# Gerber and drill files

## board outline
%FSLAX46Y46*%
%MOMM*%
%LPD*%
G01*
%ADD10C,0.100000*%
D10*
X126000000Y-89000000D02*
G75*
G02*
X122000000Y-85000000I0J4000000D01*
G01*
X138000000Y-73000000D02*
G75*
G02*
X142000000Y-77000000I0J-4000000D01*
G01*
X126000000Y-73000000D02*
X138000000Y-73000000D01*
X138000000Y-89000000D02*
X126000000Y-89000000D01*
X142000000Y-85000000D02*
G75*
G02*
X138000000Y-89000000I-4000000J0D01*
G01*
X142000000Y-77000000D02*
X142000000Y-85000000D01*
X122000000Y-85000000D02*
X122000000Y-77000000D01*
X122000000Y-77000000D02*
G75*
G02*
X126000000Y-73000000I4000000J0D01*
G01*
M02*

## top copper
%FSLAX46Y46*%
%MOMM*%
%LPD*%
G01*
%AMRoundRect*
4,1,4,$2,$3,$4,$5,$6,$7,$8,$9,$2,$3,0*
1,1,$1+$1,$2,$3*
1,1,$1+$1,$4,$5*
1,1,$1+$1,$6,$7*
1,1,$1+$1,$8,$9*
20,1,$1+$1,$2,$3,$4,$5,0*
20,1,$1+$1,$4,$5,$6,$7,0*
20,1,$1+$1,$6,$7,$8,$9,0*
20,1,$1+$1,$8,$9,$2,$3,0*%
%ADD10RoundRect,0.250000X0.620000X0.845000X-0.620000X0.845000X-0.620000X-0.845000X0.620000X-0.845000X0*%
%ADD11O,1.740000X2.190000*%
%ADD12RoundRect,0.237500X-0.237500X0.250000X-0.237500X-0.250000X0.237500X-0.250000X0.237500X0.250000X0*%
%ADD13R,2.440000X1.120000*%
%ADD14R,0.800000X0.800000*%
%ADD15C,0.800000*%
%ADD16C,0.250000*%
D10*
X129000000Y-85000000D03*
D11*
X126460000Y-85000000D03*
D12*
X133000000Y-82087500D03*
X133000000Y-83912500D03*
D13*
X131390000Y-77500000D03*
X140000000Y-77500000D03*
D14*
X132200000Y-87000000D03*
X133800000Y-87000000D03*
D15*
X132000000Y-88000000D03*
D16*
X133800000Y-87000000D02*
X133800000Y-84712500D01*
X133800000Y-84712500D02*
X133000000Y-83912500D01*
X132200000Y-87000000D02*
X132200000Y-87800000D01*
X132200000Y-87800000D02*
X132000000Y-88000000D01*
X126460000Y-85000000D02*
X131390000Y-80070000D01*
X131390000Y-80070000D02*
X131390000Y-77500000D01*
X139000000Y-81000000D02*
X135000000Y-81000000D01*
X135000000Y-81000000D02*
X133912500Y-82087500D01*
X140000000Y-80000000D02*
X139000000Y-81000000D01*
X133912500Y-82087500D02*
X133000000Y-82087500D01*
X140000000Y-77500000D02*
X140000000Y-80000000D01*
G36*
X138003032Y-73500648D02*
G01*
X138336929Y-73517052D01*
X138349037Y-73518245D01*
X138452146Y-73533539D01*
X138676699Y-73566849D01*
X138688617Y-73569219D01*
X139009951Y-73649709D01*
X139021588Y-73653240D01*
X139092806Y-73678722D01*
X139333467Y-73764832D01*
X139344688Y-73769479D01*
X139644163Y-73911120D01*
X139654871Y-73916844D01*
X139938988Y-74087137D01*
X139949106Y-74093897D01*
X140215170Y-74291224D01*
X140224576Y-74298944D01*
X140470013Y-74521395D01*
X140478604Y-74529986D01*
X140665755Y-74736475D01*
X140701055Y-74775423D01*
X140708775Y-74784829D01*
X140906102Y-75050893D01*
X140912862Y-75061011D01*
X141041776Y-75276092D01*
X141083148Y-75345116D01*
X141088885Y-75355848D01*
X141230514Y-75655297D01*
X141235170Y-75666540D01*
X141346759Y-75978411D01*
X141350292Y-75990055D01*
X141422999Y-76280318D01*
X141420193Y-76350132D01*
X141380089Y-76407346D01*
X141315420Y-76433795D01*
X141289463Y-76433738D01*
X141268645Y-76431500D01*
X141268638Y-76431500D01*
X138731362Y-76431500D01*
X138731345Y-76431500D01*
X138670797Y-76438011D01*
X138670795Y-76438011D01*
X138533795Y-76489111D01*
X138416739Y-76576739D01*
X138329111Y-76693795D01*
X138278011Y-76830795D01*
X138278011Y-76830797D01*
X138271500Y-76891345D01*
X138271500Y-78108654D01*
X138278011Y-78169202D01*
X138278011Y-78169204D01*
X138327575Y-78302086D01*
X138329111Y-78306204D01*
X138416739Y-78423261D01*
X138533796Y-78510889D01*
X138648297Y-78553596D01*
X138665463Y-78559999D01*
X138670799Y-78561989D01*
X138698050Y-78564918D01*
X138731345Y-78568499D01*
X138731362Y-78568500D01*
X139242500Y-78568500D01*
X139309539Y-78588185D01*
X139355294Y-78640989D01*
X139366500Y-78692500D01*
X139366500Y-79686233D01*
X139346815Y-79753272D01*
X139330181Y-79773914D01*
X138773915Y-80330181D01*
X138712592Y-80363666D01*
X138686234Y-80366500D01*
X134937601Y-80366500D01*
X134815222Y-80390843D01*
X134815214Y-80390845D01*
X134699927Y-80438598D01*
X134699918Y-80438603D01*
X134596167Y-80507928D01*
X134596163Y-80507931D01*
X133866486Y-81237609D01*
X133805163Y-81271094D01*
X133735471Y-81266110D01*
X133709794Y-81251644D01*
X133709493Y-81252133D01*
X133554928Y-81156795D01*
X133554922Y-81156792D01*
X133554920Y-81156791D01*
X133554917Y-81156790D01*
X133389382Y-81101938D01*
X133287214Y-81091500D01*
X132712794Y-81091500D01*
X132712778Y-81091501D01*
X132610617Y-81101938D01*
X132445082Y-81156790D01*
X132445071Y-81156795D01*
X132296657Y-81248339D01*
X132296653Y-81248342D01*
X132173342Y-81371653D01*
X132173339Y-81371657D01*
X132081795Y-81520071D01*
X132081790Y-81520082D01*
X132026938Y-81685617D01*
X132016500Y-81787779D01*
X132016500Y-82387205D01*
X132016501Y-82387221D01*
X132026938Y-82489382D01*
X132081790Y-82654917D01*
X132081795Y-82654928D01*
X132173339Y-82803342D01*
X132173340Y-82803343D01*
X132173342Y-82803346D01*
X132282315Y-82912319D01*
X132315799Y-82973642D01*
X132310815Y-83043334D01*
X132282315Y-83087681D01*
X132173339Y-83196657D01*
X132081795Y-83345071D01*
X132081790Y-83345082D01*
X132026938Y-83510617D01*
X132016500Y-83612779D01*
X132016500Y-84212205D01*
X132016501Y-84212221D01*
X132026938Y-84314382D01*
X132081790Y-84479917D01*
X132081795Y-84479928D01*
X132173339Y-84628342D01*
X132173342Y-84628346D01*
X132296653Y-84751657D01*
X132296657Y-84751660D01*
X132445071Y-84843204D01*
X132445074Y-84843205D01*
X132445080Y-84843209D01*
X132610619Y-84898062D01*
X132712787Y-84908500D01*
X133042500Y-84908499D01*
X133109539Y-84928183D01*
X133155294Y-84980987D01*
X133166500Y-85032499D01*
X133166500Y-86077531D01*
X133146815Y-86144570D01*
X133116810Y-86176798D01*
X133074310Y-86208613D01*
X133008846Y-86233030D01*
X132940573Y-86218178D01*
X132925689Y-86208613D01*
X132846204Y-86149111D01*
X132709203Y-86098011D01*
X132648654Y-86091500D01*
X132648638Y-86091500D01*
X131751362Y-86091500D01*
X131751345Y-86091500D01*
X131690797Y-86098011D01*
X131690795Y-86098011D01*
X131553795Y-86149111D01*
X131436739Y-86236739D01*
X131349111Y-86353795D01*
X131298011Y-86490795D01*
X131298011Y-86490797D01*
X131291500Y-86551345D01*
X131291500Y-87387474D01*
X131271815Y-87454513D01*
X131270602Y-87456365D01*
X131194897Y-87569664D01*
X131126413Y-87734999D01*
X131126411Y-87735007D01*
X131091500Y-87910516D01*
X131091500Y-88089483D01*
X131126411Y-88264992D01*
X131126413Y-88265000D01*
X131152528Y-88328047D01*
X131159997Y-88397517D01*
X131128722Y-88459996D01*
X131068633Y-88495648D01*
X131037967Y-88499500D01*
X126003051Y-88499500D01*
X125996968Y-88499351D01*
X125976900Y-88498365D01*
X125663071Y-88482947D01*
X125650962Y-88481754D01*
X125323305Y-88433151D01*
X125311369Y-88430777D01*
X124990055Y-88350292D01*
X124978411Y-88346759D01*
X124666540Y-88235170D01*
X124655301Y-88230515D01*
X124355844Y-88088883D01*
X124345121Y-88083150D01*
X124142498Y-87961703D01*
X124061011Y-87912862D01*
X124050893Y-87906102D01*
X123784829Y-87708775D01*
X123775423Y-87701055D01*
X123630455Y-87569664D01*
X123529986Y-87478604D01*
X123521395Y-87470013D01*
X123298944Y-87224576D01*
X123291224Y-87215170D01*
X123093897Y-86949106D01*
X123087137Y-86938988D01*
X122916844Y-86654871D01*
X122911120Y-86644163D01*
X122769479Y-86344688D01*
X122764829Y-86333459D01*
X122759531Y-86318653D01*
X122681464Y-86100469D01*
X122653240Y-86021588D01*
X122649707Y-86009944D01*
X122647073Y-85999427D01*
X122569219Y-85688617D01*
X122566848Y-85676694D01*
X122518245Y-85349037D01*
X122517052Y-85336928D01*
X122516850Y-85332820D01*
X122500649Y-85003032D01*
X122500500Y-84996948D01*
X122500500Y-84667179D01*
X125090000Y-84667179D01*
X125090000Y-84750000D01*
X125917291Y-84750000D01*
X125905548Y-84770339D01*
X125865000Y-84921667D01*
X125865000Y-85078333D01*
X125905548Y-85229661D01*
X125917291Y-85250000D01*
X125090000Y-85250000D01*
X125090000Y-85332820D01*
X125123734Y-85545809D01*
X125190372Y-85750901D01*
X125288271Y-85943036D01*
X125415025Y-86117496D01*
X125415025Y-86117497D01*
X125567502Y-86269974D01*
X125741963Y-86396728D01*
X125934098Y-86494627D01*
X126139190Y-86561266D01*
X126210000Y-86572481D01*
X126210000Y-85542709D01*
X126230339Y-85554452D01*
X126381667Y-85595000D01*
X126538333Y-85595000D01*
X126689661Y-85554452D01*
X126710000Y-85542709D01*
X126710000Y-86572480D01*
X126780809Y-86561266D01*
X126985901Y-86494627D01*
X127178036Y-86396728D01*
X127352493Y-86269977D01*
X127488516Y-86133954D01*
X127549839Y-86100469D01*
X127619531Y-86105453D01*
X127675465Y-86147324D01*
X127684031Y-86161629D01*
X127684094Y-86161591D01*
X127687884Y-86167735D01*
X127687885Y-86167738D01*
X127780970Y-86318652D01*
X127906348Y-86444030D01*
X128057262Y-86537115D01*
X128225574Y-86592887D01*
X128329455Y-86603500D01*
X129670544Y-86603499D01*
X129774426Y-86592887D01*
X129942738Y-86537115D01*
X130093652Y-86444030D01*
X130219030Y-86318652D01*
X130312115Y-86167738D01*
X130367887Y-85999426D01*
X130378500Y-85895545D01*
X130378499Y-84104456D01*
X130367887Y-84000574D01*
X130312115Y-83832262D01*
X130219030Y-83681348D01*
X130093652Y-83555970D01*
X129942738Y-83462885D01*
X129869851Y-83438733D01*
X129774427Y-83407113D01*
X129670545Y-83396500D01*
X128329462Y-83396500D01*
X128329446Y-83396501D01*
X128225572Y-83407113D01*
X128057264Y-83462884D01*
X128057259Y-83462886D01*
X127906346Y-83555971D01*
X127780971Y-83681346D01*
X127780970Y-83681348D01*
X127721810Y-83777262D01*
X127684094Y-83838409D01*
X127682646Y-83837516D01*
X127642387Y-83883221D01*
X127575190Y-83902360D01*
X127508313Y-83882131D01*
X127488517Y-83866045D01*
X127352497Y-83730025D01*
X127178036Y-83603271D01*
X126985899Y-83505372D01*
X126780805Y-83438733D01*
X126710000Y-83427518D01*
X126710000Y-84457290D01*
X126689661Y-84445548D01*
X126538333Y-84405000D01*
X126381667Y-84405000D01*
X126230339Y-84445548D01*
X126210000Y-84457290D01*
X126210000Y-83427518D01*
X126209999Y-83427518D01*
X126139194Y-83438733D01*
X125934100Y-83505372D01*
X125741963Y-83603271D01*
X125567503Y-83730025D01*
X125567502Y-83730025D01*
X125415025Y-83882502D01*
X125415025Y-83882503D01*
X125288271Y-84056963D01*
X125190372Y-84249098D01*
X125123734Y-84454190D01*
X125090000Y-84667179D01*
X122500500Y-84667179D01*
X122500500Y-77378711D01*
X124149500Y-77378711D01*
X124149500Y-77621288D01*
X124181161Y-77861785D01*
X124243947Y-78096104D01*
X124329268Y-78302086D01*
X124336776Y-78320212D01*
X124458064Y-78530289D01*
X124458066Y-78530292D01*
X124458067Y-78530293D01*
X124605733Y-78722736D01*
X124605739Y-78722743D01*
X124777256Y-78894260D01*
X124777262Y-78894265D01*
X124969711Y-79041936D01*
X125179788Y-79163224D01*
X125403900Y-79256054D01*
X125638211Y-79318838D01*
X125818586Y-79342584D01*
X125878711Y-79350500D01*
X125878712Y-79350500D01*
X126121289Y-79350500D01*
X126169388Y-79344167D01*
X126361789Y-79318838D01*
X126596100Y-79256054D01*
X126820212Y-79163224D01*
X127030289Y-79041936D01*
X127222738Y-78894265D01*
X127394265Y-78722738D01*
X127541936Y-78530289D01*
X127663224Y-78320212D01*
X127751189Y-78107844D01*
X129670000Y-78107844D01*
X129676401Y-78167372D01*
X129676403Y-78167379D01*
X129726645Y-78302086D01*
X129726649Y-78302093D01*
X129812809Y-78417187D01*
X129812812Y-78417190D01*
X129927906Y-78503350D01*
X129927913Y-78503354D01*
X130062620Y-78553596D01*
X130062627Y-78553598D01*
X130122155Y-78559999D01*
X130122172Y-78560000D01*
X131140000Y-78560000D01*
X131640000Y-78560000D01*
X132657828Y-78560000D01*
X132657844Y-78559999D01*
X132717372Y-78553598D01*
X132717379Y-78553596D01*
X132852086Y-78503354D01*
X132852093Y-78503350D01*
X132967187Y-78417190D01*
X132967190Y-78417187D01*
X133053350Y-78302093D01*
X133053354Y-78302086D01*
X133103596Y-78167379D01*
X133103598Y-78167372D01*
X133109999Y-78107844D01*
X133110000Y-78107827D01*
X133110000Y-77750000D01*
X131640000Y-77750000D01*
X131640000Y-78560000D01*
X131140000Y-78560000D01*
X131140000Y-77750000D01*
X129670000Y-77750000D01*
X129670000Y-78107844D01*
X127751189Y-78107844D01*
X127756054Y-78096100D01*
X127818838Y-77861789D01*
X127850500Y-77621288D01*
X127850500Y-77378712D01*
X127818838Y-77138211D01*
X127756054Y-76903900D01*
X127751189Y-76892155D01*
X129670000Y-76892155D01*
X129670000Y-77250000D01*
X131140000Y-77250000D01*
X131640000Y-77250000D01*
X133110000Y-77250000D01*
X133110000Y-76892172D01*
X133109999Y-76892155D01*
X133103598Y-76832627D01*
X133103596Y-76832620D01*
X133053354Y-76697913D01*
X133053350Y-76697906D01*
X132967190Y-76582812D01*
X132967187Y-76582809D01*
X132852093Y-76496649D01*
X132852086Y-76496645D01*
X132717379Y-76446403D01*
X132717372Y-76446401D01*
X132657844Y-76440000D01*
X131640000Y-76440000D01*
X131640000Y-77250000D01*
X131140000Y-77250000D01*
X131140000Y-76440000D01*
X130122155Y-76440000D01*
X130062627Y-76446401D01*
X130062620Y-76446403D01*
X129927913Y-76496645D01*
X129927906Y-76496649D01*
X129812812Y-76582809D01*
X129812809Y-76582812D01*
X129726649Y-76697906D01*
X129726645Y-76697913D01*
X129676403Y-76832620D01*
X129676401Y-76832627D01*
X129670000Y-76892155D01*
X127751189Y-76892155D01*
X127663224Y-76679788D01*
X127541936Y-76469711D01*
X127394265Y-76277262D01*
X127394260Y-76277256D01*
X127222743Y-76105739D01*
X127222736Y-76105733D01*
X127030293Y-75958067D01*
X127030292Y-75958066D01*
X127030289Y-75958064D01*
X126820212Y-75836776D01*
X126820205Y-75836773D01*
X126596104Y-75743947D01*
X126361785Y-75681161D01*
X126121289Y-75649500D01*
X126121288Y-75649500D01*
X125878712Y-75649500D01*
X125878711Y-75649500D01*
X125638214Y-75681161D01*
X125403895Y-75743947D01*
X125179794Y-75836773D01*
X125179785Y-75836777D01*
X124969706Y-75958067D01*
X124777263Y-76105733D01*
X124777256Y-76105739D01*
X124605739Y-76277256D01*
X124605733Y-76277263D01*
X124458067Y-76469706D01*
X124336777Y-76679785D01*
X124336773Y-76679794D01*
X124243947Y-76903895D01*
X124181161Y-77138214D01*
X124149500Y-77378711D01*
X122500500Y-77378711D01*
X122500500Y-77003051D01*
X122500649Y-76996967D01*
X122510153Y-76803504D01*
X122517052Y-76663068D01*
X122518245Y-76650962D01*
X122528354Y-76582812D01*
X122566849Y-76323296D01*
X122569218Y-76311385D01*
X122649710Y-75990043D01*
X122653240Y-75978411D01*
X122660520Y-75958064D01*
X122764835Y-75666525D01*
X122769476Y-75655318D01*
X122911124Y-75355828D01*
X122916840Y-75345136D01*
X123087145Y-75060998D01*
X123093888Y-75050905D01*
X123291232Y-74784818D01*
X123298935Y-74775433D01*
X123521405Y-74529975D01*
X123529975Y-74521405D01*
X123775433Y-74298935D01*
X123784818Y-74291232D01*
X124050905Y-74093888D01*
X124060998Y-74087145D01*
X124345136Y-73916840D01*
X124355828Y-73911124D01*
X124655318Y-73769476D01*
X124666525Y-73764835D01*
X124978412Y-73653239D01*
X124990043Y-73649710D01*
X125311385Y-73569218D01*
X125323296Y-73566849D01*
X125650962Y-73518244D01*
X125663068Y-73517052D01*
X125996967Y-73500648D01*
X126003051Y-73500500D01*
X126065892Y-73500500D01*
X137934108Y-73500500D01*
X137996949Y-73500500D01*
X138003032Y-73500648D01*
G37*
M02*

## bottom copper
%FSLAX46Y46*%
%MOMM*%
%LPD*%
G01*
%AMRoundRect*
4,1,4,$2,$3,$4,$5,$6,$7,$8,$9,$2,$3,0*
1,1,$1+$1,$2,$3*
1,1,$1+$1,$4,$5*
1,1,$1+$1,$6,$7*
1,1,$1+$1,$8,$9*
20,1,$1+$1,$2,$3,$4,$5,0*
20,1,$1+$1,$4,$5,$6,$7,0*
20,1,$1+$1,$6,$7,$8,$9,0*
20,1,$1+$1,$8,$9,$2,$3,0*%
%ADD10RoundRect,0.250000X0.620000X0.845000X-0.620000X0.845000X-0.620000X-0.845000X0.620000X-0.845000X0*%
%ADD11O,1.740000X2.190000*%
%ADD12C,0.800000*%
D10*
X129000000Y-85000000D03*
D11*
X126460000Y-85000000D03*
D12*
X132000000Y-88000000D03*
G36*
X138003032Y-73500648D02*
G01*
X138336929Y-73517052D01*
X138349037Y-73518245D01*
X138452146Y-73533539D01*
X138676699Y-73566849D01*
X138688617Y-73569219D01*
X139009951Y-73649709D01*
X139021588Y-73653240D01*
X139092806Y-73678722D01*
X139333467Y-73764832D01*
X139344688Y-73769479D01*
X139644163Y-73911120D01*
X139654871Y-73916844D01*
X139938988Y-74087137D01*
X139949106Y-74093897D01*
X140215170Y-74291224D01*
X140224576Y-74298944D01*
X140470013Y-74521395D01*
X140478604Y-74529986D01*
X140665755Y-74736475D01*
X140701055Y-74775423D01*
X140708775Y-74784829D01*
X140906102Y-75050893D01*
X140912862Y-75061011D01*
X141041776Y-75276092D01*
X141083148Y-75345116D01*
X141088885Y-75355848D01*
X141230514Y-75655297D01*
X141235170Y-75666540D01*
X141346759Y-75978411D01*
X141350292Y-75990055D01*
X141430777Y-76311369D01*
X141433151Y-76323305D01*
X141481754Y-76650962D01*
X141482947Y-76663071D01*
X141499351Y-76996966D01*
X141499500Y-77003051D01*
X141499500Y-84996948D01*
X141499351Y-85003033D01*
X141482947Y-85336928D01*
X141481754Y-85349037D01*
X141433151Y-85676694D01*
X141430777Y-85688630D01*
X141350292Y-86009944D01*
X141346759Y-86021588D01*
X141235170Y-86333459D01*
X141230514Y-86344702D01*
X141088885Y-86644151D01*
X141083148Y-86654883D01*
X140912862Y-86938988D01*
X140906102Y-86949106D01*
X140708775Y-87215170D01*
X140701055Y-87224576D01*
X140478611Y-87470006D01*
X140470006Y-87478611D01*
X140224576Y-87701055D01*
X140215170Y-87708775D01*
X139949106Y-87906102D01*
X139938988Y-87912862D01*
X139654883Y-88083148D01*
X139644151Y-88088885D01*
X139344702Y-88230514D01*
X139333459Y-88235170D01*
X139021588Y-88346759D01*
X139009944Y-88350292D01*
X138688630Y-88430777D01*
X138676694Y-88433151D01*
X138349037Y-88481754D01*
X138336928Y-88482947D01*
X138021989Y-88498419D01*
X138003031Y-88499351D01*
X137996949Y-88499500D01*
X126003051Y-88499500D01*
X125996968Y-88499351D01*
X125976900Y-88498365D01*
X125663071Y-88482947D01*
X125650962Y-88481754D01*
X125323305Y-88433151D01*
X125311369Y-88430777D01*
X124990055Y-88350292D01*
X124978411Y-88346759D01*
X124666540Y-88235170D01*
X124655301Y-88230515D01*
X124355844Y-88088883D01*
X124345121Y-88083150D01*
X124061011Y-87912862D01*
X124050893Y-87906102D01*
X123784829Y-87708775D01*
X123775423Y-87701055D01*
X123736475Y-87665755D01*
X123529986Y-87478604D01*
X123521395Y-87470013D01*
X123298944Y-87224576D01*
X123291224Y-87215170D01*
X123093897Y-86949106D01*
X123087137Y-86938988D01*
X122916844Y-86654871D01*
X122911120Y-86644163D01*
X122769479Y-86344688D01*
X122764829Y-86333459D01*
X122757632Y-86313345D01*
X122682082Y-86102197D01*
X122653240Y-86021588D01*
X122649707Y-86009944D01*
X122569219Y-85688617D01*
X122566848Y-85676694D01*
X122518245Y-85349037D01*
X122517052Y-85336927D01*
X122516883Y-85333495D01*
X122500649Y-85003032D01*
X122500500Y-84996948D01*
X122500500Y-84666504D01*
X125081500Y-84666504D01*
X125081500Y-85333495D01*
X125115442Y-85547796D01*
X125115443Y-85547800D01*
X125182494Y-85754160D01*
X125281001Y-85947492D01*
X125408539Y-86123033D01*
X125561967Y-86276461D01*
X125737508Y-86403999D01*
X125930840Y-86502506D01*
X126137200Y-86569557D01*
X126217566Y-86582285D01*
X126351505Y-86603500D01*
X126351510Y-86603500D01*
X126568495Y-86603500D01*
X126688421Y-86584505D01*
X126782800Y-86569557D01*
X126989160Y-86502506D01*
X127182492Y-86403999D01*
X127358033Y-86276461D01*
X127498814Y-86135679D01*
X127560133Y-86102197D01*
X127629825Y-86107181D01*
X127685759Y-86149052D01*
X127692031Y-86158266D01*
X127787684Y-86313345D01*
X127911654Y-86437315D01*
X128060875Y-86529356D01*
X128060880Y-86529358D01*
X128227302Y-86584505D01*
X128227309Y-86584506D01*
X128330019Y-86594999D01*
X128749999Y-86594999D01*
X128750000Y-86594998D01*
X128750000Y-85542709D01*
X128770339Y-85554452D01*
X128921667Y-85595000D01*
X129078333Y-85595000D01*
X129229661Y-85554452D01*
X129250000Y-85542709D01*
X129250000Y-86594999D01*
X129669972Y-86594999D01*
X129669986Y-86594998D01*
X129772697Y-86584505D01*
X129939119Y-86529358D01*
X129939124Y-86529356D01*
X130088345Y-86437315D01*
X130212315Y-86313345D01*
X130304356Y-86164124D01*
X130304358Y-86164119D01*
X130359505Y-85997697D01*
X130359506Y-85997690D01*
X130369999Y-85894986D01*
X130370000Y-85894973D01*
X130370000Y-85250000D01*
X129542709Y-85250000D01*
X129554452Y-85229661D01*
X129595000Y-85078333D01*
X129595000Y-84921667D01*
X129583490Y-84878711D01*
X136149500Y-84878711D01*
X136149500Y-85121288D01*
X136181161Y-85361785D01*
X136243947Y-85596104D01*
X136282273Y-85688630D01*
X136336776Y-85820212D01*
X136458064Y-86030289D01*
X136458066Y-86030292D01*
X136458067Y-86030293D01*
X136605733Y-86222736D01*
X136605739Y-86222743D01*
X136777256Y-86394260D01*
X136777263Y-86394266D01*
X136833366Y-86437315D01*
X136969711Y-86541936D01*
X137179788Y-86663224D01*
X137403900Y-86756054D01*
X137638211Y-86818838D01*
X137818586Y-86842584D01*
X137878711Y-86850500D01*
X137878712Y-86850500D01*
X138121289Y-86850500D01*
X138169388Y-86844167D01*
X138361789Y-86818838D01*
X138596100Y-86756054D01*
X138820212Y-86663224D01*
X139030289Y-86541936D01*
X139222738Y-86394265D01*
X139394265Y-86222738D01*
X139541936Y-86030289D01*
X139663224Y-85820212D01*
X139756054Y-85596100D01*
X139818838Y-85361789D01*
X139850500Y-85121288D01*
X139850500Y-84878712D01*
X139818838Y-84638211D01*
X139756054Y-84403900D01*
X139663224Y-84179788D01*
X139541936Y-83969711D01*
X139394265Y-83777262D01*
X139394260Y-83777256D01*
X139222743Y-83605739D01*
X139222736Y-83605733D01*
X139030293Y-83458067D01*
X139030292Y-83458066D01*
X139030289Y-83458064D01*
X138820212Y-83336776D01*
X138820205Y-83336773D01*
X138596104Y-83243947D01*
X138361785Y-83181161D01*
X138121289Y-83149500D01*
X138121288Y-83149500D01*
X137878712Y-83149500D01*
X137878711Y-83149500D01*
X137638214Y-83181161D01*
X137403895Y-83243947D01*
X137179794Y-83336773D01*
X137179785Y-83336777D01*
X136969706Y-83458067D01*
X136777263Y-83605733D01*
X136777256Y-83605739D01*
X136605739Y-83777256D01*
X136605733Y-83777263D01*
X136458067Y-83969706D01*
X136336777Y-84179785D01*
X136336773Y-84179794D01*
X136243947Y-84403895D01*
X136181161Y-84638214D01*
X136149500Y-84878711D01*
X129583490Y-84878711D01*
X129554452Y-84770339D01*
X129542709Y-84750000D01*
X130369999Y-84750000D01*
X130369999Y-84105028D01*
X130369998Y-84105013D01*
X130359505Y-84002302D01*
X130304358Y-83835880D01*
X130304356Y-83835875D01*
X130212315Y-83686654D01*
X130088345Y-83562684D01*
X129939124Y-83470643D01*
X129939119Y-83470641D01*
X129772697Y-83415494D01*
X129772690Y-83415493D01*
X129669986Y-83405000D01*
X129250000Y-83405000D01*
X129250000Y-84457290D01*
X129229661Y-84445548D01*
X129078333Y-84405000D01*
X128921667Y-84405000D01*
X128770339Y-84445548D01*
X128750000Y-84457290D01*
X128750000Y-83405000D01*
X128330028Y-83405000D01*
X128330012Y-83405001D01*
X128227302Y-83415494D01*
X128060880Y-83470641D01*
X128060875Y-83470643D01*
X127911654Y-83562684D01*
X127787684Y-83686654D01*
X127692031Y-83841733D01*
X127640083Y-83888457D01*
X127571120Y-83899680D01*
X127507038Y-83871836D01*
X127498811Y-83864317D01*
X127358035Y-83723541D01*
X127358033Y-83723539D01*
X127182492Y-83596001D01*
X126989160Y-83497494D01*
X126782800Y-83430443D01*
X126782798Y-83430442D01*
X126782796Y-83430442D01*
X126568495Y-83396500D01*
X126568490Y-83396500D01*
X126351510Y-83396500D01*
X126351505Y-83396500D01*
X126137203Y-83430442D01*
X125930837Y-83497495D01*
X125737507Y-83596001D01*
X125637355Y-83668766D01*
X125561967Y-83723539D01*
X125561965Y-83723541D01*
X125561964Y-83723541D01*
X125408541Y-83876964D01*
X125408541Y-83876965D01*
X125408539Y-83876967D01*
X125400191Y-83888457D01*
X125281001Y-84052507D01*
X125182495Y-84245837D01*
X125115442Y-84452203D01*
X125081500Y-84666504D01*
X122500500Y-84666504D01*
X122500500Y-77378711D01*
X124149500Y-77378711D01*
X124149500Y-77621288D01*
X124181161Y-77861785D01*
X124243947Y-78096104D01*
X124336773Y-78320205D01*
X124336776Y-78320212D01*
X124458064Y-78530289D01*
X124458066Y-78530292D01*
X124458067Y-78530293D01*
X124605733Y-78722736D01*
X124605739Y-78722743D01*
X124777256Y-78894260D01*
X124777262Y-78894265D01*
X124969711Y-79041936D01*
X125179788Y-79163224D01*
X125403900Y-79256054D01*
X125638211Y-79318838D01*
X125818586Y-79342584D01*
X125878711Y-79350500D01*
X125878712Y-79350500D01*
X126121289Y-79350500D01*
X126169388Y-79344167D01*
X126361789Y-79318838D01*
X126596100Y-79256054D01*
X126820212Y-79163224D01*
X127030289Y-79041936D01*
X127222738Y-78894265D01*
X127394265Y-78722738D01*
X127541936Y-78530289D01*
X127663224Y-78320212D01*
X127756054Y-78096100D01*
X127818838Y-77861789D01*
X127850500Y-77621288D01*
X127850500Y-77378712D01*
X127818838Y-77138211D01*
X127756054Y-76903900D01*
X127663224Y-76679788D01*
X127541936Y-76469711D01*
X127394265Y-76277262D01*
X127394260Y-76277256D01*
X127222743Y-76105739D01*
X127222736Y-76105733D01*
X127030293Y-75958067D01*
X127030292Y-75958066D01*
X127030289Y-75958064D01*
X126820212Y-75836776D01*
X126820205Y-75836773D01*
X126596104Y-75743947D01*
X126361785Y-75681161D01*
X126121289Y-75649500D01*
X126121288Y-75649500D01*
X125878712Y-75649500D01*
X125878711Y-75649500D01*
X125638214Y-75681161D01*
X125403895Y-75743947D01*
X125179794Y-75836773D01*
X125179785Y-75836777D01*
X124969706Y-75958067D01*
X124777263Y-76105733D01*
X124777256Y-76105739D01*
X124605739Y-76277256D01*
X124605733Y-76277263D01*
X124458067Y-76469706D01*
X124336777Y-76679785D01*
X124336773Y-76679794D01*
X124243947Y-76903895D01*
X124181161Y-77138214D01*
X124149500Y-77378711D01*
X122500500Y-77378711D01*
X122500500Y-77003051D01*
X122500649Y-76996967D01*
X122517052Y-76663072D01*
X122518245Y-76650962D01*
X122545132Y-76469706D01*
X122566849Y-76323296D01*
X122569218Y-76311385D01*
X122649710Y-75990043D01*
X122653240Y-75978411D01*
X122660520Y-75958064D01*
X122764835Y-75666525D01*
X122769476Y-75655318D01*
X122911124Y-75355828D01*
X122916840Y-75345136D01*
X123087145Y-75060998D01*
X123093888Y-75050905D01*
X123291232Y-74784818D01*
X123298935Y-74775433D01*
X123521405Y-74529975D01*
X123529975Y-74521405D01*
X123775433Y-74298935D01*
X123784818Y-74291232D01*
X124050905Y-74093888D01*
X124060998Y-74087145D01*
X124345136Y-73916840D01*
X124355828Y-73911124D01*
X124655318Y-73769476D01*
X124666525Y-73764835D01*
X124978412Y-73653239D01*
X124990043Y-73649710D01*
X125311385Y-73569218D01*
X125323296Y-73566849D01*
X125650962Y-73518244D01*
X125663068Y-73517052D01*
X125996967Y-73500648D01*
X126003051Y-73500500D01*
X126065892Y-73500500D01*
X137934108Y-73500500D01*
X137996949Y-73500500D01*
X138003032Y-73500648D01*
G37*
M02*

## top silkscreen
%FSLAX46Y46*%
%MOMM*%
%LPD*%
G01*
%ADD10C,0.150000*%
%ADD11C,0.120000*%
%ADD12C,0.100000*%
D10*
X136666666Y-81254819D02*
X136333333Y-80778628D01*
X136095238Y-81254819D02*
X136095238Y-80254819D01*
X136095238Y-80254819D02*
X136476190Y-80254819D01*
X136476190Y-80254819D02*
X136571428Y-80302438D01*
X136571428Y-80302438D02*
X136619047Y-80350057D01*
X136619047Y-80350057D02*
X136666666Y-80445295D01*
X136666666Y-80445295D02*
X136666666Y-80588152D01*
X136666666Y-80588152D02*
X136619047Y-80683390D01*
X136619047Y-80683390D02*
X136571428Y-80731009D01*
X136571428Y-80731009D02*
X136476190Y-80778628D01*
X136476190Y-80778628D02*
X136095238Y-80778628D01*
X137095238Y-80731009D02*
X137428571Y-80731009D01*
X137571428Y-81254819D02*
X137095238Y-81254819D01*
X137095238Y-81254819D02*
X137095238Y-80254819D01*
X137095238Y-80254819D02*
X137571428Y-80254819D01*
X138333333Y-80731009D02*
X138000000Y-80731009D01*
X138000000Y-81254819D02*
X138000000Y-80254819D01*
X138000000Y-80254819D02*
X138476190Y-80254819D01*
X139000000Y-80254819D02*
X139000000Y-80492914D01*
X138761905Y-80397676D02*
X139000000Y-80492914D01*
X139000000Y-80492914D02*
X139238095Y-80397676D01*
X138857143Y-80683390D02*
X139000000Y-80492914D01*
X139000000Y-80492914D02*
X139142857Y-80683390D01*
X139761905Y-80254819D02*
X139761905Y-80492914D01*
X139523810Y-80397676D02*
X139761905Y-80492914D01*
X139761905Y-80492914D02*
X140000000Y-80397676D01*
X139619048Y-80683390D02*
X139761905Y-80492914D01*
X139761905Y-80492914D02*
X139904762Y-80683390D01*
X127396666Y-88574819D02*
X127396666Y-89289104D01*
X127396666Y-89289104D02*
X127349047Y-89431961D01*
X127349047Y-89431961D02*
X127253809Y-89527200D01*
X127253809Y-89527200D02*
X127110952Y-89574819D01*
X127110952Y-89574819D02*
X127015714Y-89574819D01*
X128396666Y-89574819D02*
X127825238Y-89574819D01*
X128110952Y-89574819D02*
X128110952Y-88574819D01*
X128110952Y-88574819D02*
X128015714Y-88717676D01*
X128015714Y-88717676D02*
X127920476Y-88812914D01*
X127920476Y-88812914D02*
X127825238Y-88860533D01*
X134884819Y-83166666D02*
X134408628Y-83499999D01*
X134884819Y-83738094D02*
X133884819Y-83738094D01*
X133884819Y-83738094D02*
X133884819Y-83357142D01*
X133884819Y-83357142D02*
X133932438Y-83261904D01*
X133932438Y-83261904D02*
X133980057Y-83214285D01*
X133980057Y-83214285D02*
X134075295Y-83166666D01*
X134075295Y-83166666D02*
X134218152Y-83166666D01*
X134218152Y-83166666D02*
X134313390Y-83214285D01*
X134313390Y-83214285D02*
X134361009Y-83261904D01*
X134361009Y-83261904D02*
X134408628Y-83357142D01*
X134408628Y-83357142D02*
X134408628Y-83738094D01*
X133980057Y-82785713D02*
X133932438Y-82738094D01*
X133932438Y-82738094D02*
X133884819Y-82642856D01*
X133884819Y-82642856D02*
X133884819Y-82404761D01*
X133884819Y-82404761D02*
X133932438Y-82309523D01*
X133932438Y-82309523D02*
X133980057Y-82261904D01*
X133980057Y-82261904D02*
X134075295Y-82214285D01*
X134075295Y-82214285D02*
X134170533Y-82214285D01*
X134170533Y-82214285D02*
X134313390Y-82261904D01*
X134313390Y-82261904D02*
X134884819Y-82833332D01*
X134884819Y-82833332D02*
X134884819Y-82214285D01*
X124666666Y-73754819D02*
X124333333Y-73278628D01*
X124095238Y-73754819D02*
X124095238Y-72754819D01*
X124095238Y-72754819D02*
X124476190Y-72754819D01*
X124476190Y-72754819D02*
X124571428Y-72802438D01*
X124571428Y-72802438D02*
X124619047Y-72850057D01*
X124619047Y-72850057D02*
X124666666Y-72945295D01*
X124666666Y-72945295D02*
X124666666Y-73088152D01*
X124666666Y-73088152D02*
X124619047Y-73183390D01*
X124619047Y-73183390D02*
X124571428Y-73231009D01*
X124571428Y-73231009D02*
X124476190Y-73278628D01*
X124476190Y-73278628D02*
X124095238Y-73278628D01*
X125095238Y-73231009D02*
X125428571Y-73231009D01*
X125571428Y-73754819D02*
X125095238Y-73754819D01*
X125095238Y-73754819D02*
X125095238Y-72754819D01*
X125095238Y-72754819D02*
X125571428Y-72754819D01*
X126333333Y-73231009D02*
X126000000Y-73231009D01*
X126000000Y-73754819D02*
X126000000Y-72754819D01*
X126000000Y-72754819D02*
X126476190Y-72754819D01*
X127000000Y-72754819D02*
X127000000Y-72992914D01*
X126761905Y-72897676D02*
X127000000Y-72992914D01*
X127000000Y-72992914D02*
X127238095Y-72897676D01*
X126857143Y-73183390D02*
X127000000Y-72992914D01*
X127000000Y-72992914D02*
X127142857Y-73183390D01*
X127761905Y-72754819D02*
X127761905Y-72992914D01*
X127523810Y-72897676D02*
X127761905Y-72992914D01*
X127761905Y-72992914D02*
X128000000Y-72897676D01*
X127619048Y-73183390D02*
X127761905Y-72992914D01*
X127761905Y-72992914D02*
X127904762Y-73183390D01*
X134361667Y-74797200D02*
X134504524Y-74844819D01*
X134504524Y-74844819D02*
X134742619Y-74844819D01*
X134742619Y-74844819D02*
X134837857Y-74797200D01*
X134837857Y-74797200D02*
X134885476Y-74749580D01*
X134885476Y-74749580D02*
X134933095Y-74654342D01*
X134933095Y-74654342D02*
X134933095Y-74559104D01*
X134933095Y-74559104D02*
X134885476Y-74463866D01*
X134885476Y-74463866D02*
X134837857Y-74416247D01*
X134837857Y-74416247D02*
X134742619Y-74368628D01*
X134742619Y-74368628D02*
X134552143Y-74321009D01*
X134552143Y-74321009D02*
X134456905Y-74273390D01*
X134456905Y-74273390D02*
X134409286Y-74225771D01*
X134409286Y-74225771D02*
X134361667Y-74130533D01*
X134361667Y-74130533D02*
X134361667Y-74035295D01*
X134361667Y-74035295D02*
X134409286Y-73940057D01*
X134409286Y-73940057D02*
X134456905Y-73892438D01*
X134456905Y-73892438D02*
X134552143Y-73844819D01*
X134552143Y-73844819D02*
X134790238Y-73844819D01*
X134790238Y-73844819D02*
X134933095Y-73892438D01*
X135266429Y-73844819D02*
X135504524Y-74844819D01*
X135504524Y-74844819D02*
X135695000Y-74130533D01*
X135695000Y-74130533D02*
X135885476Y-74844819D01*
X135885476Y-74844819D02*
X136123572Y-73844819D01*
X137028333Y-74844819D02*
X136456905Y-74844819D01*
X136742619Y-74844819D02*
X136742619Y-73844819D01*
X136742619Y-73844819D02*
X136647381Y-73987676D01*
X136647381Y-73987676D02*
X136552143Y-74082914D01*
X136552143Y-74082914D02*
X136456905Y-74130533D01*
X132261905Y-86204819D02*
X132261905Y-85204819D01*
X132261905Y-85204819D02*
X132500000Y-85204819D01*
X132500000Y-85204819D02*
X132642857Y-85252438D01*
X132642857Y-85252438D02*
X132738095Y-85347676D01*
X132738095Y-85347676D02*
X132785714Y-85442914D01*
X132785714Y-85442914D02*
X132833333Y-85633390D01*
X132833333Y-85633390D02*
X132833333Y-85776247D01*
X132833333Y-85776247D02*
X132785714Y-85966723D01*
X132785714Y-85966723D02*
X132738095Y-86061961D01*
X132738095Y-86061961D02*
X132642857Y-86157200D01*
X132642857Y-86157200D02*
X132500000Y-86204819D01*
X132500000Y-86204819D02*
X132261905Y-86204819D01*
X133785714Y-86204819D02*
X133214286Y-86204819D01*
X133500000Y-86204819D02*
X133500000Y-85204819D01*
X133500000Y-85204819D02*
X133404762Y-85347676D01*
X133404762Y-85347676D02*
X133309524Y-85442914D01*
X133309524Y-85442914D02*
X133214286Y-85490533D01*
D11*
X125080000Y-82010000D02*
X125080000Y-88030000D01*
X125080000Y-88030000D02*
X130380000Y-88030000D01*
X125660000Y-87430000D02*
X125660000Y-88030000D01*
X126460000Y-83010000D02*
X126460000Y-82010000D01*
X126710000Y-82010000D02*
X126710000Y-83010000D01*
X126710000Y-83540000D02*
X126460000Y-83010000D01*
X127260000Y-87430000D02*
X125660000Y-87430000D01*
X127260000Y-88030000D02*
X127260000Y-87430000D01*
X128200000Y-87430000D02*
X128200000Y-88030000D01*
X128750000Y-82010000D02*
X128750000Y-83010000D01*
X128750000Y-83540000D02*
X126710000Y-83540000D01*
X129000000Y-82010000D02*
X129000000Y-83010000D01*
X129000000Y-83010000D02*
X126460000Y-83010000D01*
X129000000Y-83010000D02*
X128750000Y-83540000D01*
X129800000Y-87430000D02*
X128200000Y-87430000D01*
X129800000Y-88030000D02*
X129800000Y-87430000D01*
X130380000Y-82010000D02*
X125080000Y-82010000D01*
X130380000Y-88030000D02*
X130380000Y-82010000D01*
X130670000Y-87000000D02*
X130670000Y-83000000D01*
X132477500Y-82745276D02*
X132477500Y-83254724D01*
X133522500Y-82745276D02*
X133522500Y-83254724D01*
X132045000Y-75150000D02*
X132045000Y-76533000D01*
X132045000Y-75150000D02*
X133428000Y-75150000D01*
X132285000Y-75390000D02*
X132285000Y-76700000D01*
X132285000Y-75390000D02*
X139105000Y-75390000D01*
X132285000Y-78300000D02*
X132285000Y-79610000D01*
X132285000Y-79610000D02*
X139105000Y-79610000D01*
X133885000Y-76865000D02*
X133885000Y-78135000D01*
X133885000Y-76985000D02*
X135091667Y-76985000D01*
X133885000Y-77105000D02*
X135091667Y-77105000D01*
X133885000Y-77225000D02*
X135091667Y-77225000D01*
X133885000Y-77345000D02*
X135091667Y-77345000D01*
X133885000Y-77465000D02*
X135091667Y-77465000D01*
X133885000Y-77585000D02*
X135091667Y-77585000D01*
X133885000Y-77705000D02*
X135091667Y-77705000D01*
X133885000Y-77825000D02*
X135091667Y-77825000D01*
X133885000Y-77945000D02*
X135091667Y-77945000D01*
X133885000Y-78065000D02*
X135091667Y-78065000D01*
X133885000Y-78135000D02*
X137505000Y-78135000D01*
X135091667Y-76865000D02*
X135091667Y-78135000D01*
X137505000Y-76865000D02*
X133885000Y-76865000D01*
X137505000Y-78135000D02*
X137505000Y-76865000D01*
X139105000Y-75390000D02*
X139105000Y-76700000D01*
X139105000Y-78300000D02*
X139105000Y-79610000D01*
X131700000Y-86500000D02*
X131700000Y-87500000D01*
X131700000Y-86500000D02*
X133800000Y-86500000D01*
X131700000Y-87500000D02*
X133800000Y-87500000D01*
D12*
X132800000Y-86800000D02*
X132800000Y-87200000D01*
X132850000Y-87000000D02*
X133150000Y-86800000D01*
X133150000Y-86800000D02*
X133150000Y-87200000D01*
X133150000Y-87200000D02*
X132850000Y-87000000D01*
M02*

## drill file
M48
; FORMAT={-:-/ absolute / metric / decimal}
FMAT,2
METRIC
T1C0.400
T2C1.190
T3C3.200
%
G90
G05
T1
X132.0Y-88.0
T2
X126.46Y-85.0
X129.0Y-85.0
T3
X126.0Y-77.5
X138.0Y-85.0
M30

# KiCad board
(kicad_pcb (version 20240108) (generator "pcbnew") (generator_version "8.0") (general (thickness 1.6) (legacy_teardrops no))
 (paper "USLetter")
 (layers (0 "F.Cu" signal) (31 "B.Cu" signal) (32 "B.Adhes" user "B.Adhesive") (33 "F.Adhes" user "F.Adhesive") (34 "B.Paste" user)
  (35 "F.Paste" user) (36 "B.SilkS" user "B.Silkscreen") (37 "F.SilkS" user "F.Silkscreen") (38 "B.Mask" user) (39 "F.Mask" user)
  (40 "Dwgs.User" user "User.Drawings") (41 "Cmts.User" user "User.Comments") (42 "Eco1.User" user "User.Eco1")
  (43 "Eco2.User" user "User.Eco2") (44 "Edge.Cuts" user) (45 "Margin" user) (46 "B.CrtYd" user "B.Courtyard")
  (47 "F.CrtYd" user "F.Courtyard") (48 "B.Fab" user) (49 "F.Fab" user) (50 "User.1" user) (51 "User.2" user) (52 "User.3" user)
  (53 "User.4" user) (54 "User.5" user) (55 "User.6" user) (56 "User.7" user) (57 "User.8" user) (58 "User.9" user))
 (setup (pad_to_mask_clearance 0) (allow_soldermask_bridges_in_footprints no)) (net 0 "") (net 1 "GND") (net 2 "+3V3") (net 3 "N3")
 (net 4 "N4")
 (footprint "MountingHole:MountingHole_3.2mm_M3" (layer "F.Cu") (at 138 85)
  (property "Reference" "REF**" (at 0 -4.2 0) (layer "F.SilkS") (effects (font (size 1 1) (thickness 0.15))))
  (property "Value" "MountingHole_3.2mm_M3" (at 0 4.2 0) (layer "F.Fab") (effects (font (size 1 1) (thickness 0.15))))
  (pad "" np_thru_hole circle (at 0 0) (size 3.2 3.2) (drill 3.2) (layers "*.Cu" "*.Mask")))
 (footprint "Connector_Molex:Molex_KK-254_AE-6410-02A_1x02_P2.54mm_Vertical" (layer "F.Cu") (at 129 85 180)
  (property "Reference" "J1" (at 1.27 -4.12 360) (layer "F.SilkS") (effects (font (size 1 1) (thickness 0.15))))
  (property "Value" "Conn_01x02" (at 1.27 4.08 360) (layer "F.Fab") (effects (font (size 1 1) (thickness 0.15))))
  (fp_line (start 3.92 2.99) (end 3.92 -3.03) (stroke (width 0.12) (type solid)) (layer "F.SilkS"))
  (fp_line (start 3.92 -3.03) (end -1.38 -3.03) (stroke (width 0.12) (type solid)) (layer "F.SilkS"))
  (fp_line (start 3.34 -2.43) (end 3.34 -3.03) (stroke (width 0.12) (type solid)) (layer "F.SilkS"))
  (fp_line (start 2.54 1.99) (end 2.54 2.99) (stroke (width 0.12) (type solid)) (layer "F.SilkS"))
  (fp_line (start 2.29 2.99) (end 2.29 1.99) (stroke (width 0.12) (type solid)) (layer "F.SilkS"))
  (fp_line (start 2.29 1.46) (end 2.54 1.99) (stroke (width 0.12) (type solid)) (layer "F.SilkS"))
  (fp_line (start 1.74 -2.43) (end 3.34 -2.43) (stroke (width 0.12) (type solid)) (layer "F.SilkS"))
  (fp_line (start 1.74 -3.03) (end 1.74 -2.43) (stroke (width 0.12) (type solid)) (layer "F.SilkS"))
  (fp_line (start 0.8 -2.43) (end 0.8 -3.03) (stroke (width 0.12) (type solid)) (layer "F.SilkS"))
  (fp_line (start 0.25 2.99) (end 0.25 1.99) (stroke (width 0.12) (type solid)) (layer "F.SilkS"))
  (fp_line (start 0.25 1.46) (end 2.29 1.46) (stroke (width 0.12) (type solid)) (layer "F.SilkS"))
  (fp_line (start 0 2.99) (end 0 1.99) (stroke (width 0.12) (type solid)) (layer "F.SilkS"))
  (fp_line (start 0 1.99) (end 2.54 1.99) (stroke (width 0.12) (type solid)) (layer "F.SilkS"))
  (fp_line (start 0 1.99) (end 0.25 1.46) (stroke (width 0.12) (type solid)) (layer "F.SilkS"))
  (fp_line (start -0.8 -2.43) (end 0.8 -2.43) (stroke (width 0.12) (type solid)) (layer "F.SilkS"))
  (fp_line (start -0.8 -3.03) (end -0.8 -2.43) (stroke (width 0.12) (type solid)) (layer "F.SilkS"))
  (fp_line (start -1.38 2.99) (end 3.92 2.99) (stroke (width 0.12) (type solid)) (layer "F.SilkS"))
  (fp_line (start -1.38 -3.03) (end -1.38 2.99) (stroke (width 0.12) (type solid)) (layer "F.SilkS"))
  (fp_line (start -1.67 -2) (end -1.67 2) (stroke (width 0.12) (type solid)) (layer "F.SilkS"))
  (pad "1" thru_hole roundrect (at 0 0 180) (size 1.74 2.19) (drill 1.19) (layers "*.Cu" "*.Mask") (remove_unused_layers no)
   (roundrect_rratio 0.143678) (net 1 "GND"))
  (pad "2" thru_hole oval (at 2.54 0 180) (size 1.74 2.19) (drill 1.19) (layers "*.Cu" "*.Mask") (remove_unused_layers no) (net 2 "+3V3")))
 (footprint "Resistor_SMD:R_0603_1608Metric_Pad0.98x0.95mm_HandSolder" (layer "F.Cu") (at 133 83 -90)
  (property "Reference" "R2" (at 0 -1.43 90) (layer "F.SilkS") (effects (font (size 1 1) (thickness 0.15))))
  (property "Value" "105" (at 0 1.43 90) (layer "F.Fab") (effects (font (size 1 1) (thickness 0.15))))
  (fp_line (start -0.254724 0.5225) (end 0.254724 0.5225) (stroke (width 0.12) (type solid)) (layer "F.SilkS"))
  (fp_line (start -0.254724 -0.5225) (end 0.254724 -0.5225) (stroke (width 0.12) (type solid)) (layer "F.SilkS"))
  (pad "1" smd roundrect (at -0.9125 0 270) (size 0.975 0.95) (layers "F.Cu" "F.Paste" "F.Mask") (roundrect_rratio 0.25) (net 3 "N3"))
  (pad "2" smd roundrect (at 0.9125 0 270) (size 0.975 0.95) (layers "F.Cu" "F.Paste" "F.Mask") (roundrect_rratio 0.25) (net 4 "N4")))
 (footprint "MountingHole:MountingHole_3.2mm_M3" (layer "F.Cu") (at 126 77.5)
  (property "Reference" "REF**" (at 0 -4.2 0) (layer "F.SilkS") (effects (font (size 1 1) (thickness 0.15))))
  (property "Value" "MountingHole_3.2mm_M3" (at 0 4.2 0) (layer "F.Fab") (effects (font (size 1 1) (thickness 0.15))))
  (pad "" np_thru_hole circle (at 0 0) (size 3.2 3.2) (drill 3.2) (layers "*.Cu" "*.Mask")))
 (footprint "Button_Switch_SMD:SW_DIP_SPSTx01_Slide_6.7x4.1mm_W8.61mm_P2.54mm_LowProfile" (layer "F.Cu") (at 135.695 77.5)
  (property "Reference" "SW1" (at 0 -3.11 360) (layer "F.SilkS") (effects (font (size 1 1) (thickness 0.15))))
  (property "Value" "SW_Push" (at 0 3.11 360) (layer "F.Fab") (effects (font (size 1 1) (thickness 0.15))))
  (fp_line (start -3.65 -2.35) (end -3.65 -0.967) (stroke (width 0.12) (type solid)) (layer "F.SilkS"))
  (fp_line (start -3.65 -2.35) (end -2.267 -2.35) (stroke (width 0.12) (type solid)) (layer "F.SilkS"))
  (fp_line (start -3.41 -2.11) (end -3.41 -0.8) (stroke (width 0.12) (type solid)) (layer "F.SilkS"))
  (fp_line (start -3.41 -2.11) (end 3.41 -2.11) (stroke (width 0.12) (type solid)) (layer "F.SilkS"))
  (fp_line (start -3.41 0.8) (end -3.41 2.11) (stroke (width 0.12) (type solid)) (layer "F.SilkS"))
  (fp_line (start -3.41 2.11) (end 3.41 2.11) (stroke (width 0.12) (type solid)) (layer "F.SilkS"))
  (fp_line (start -1.81 -0.635) (end -1.81 0.635) (stroke (width 0.12) (type solid)) (layer "F.SilkS"))
  (fp_line (start -1.81 -0.515) (end -0.603333 -0.515) (stroke (width 0.12) (type solid)) (layer "F.SilkS"))
  (fp_line (start -1.81 -0.395) (end -0.603333 -0.395) (stroke (width 0.12) (type solid)) (layer "F.SilkS"))
  (fp_line (start -1.81 -0.275) (end -0.603333 -0.275) (stroke (width 0.12) (type solid)) (layer "F.SilkS"))
  (fp_line (start -1.81 -0.155) (end -0.603333 -0.155) (stroke (width 0.12) (type solid)) (layer "F.SilkS"))
  (fp_line (start -1.81 -0.035) (end -0.603333 -0.035) (stroke (width 0.12) (type solid)) (layer "F.SilkS"))
  (fp_line (start -1.81 0.085) (end -0.603333 0.085) (stroke (width 0.12) (type solid)) (layer "F.SilkS"))
  (fp_line (start -1.81 0.205) (end -0.603333 0.205) (stroke (width 0.12) (type solid)) (layer "F.SilkS"))
  (fp_line (start -1.81 0.325) (end -0.603333 0.325) (stroke (width 0.12) (type solid)) (layer "F.SilkS"))
  (fp_line (start -1.81 0.445) (end -0.603333 0.445) (stroke (width 0.12) (type solid)) (layer "F.SilkS"))
  (fp_line (start -1.81 0.565) (end -0.603333 0.565) (stroke (width 0.12) (type solid)) (layer "F.SilkS"))
  (fp_line (start -1.81 0.635) (end 1.81 0.635) (stroke (width 0.12) (type solid)) (layer "F.SilkS"))
  (fp_line (start -0.603333 -0.635) (end -0.603333 0.635) (stroke (width 0.12) (type solid)) (layer "F.SilkS"))
  (fp_line (start 1.81 -0.635) (end -1.81 -0.635) (stroke (width 0.12) (type solid)) (layer "F.SilkS"))
  (fp_line (start 1.81 0.635) (end 1.81 -0.635) (stroke (width 0.12) (type solid)) (layer "F.SilkS"))
  (fp_line (start 3.41 -2.11) (end 3.41 -0.8) (stroke (width 0.12) (type solid)) (layer "F.SilkS"))
  (fp_line (start 3.41 0.8) (end 3.41 2.11) (stroke (width 0.12) (type solid)) (layer "F.SilkS"))
  (pad "1" smd rect (at -4.305 0) (size 2.44 1.12) (layers "F.Cu" "F.Paste" "F.Mask") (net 2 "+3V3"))
  (pad "2" smd rect (at 4.305 0) (size 2.44 1.12) (layers "F.Cu" "F.Paste" "F.Mask") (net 3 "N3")))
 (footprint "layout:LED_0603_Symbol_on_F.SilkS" (layer "F.Cu") (at 133 87)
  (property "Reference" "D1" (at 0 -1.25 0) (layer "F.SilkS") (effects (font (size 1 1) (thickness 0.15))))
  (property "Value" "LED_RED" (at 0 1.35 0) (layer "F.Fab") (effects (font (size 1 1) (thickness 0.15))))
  (fp_line (start -1.3 -0.5) (end -1.3 0.5) (stroke (width 0.12) (type solid)) (layer "F.SilkS"))
  (fp_line (start -1.3 -0.5) (end 0.8 -0.5) (stroke (width 0.12) (type solid)) (layer "F.SilkS"))
  (fp_line (start -1.3 0.5) (end 0.8 0.5) (stroke (width 0.12) (type solid)) (layer "F.SilkS"))
  (fp_line (start -0.2 -0.2) (end -0.2 0.2) (stroke (width 0.1) (type solid)) (layer "F.SilkS"))
  (fp_line (start -0.15 0) (end 0.15 -0.2) (stroke (width 0.1) (type solid)) (layer "F.SilkS"))
  (fp_line (start 0.15 -0.2) (end 0.15 0.2) (stroke (width 0.1) (type solid)) (layer "F.SilkS"))
  (fp_line (start 0.15 0.2) (end -0.15 0) (stroke (width 0.1) (type solid)) (layer "F.SilkS"))
  (pad "1" smd rect (at -0.8 0 180) (size 0.8 0.8) (layers "F.Cu" "F.Paste" "F.Mask") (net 1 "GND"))
  (pad "2" smd rect (at 0.8 0 180) (size 0.8 0.8) (layers "F.Cu" "F.Paste" "F.Mask") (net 4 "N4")))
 (gr_arc (start 126 89) (mid 123.171573 87.828427) (end 122 85) (stroke (width 0.1) (type default)) (layer "Edge.Cuts"))
 (gr_arc (start 138 73) (mid 140.828427 74.171573) (end 142 77) (stroke (width 0.1) (type default)) (layer "Edge.Cuts"))
 (gr_line (start 126 73) (end 138 73) (stroke (width 0.1) (type default)) (layer "Edge.Cuts"))
 (gr_line (start 138 89) (end 126 89) (stroke (width 0.1) (type default)) (layer "Edge.Cuts"))
 (gr_arc (start 142 85) (mid 140.828427 87.828427) (end 138 89) (stroke (width 0.1) (type default)) (layer "Edge.Cuts"))
 (gr_line (start 142 77) (end 142 85) (stroke (width 0.1) (type default)) (layer "Edge.Cuts"))
 (gr_line (start 122 85) (end 122 77) (stroke (width 0.1) (type default)) (layer "Edge.Cuts"))
 (gr_arc (start 122 77) (mid 123.171573 74.171573) (end 126 73) (stroke (width 0.1) (type default)) (layer "Edge.Cuts"))
 (segment (start 133.8 87) (end 133.8 84.7125) (width 0.25) (layer "F.Cu") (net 4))
 (segment (start 133.8 84.7125) (end 133 83.9125) (width 0.25) (layer "F.Cu") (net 4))
 (segment (start 132.2 87) (end 132.2 87.8) (width 0.25) (layer "F.Cu") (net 1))
 (segment (start 132.2 87.8) (end 132 88) (width 0.25) (layer "F.Cu") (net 1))
 (via (at 132 88) (size 0.8) (drill 0.4) (layers "F.Cu" "B.Cu") (free yes) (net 1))
 (segment (start 126.46 85) (end 131.39 80.07) (width 0.25) (layer "F.Cu") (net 2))
 (segment (start 131.39 80.07) (end 131.39 77.5) (width 0.25) (layer "F.Cu") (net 2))
 (segment (start 139 81) (end 135 81) (width 0.25) (layer "F.Cu") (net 3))
 (segment (start 135 81) (end 133.9125 82.0875) (width 0.25) (layer "F.Cu") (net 3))
 (segment (start 140 80) (end 139 81) (width 0.25) (layer "F.Cu") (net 3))
 (segment (start 133.9125 82.0875) (end 133 82.0875) (width 0.25) (layer "F.Cu") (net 3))
 (segment (start 140 77.5) (end 140 80) (width 0.25) (layer "F.Cu") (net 3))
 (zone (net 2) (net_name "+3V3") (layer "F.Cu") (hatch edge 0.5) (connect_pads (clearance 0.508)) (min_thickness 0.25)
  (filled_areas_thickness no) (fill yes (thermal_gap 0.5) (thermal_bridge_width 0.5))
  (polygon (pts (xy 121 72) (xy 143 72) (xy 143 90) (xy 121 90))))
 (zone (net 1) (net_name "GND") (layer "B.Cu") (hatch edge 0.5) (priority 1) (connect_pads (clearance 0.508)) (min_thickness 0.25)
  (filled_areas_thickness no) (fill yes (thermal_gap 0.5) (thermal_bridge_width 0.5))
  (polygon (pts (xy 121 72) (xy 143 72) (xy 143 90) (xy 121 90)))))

